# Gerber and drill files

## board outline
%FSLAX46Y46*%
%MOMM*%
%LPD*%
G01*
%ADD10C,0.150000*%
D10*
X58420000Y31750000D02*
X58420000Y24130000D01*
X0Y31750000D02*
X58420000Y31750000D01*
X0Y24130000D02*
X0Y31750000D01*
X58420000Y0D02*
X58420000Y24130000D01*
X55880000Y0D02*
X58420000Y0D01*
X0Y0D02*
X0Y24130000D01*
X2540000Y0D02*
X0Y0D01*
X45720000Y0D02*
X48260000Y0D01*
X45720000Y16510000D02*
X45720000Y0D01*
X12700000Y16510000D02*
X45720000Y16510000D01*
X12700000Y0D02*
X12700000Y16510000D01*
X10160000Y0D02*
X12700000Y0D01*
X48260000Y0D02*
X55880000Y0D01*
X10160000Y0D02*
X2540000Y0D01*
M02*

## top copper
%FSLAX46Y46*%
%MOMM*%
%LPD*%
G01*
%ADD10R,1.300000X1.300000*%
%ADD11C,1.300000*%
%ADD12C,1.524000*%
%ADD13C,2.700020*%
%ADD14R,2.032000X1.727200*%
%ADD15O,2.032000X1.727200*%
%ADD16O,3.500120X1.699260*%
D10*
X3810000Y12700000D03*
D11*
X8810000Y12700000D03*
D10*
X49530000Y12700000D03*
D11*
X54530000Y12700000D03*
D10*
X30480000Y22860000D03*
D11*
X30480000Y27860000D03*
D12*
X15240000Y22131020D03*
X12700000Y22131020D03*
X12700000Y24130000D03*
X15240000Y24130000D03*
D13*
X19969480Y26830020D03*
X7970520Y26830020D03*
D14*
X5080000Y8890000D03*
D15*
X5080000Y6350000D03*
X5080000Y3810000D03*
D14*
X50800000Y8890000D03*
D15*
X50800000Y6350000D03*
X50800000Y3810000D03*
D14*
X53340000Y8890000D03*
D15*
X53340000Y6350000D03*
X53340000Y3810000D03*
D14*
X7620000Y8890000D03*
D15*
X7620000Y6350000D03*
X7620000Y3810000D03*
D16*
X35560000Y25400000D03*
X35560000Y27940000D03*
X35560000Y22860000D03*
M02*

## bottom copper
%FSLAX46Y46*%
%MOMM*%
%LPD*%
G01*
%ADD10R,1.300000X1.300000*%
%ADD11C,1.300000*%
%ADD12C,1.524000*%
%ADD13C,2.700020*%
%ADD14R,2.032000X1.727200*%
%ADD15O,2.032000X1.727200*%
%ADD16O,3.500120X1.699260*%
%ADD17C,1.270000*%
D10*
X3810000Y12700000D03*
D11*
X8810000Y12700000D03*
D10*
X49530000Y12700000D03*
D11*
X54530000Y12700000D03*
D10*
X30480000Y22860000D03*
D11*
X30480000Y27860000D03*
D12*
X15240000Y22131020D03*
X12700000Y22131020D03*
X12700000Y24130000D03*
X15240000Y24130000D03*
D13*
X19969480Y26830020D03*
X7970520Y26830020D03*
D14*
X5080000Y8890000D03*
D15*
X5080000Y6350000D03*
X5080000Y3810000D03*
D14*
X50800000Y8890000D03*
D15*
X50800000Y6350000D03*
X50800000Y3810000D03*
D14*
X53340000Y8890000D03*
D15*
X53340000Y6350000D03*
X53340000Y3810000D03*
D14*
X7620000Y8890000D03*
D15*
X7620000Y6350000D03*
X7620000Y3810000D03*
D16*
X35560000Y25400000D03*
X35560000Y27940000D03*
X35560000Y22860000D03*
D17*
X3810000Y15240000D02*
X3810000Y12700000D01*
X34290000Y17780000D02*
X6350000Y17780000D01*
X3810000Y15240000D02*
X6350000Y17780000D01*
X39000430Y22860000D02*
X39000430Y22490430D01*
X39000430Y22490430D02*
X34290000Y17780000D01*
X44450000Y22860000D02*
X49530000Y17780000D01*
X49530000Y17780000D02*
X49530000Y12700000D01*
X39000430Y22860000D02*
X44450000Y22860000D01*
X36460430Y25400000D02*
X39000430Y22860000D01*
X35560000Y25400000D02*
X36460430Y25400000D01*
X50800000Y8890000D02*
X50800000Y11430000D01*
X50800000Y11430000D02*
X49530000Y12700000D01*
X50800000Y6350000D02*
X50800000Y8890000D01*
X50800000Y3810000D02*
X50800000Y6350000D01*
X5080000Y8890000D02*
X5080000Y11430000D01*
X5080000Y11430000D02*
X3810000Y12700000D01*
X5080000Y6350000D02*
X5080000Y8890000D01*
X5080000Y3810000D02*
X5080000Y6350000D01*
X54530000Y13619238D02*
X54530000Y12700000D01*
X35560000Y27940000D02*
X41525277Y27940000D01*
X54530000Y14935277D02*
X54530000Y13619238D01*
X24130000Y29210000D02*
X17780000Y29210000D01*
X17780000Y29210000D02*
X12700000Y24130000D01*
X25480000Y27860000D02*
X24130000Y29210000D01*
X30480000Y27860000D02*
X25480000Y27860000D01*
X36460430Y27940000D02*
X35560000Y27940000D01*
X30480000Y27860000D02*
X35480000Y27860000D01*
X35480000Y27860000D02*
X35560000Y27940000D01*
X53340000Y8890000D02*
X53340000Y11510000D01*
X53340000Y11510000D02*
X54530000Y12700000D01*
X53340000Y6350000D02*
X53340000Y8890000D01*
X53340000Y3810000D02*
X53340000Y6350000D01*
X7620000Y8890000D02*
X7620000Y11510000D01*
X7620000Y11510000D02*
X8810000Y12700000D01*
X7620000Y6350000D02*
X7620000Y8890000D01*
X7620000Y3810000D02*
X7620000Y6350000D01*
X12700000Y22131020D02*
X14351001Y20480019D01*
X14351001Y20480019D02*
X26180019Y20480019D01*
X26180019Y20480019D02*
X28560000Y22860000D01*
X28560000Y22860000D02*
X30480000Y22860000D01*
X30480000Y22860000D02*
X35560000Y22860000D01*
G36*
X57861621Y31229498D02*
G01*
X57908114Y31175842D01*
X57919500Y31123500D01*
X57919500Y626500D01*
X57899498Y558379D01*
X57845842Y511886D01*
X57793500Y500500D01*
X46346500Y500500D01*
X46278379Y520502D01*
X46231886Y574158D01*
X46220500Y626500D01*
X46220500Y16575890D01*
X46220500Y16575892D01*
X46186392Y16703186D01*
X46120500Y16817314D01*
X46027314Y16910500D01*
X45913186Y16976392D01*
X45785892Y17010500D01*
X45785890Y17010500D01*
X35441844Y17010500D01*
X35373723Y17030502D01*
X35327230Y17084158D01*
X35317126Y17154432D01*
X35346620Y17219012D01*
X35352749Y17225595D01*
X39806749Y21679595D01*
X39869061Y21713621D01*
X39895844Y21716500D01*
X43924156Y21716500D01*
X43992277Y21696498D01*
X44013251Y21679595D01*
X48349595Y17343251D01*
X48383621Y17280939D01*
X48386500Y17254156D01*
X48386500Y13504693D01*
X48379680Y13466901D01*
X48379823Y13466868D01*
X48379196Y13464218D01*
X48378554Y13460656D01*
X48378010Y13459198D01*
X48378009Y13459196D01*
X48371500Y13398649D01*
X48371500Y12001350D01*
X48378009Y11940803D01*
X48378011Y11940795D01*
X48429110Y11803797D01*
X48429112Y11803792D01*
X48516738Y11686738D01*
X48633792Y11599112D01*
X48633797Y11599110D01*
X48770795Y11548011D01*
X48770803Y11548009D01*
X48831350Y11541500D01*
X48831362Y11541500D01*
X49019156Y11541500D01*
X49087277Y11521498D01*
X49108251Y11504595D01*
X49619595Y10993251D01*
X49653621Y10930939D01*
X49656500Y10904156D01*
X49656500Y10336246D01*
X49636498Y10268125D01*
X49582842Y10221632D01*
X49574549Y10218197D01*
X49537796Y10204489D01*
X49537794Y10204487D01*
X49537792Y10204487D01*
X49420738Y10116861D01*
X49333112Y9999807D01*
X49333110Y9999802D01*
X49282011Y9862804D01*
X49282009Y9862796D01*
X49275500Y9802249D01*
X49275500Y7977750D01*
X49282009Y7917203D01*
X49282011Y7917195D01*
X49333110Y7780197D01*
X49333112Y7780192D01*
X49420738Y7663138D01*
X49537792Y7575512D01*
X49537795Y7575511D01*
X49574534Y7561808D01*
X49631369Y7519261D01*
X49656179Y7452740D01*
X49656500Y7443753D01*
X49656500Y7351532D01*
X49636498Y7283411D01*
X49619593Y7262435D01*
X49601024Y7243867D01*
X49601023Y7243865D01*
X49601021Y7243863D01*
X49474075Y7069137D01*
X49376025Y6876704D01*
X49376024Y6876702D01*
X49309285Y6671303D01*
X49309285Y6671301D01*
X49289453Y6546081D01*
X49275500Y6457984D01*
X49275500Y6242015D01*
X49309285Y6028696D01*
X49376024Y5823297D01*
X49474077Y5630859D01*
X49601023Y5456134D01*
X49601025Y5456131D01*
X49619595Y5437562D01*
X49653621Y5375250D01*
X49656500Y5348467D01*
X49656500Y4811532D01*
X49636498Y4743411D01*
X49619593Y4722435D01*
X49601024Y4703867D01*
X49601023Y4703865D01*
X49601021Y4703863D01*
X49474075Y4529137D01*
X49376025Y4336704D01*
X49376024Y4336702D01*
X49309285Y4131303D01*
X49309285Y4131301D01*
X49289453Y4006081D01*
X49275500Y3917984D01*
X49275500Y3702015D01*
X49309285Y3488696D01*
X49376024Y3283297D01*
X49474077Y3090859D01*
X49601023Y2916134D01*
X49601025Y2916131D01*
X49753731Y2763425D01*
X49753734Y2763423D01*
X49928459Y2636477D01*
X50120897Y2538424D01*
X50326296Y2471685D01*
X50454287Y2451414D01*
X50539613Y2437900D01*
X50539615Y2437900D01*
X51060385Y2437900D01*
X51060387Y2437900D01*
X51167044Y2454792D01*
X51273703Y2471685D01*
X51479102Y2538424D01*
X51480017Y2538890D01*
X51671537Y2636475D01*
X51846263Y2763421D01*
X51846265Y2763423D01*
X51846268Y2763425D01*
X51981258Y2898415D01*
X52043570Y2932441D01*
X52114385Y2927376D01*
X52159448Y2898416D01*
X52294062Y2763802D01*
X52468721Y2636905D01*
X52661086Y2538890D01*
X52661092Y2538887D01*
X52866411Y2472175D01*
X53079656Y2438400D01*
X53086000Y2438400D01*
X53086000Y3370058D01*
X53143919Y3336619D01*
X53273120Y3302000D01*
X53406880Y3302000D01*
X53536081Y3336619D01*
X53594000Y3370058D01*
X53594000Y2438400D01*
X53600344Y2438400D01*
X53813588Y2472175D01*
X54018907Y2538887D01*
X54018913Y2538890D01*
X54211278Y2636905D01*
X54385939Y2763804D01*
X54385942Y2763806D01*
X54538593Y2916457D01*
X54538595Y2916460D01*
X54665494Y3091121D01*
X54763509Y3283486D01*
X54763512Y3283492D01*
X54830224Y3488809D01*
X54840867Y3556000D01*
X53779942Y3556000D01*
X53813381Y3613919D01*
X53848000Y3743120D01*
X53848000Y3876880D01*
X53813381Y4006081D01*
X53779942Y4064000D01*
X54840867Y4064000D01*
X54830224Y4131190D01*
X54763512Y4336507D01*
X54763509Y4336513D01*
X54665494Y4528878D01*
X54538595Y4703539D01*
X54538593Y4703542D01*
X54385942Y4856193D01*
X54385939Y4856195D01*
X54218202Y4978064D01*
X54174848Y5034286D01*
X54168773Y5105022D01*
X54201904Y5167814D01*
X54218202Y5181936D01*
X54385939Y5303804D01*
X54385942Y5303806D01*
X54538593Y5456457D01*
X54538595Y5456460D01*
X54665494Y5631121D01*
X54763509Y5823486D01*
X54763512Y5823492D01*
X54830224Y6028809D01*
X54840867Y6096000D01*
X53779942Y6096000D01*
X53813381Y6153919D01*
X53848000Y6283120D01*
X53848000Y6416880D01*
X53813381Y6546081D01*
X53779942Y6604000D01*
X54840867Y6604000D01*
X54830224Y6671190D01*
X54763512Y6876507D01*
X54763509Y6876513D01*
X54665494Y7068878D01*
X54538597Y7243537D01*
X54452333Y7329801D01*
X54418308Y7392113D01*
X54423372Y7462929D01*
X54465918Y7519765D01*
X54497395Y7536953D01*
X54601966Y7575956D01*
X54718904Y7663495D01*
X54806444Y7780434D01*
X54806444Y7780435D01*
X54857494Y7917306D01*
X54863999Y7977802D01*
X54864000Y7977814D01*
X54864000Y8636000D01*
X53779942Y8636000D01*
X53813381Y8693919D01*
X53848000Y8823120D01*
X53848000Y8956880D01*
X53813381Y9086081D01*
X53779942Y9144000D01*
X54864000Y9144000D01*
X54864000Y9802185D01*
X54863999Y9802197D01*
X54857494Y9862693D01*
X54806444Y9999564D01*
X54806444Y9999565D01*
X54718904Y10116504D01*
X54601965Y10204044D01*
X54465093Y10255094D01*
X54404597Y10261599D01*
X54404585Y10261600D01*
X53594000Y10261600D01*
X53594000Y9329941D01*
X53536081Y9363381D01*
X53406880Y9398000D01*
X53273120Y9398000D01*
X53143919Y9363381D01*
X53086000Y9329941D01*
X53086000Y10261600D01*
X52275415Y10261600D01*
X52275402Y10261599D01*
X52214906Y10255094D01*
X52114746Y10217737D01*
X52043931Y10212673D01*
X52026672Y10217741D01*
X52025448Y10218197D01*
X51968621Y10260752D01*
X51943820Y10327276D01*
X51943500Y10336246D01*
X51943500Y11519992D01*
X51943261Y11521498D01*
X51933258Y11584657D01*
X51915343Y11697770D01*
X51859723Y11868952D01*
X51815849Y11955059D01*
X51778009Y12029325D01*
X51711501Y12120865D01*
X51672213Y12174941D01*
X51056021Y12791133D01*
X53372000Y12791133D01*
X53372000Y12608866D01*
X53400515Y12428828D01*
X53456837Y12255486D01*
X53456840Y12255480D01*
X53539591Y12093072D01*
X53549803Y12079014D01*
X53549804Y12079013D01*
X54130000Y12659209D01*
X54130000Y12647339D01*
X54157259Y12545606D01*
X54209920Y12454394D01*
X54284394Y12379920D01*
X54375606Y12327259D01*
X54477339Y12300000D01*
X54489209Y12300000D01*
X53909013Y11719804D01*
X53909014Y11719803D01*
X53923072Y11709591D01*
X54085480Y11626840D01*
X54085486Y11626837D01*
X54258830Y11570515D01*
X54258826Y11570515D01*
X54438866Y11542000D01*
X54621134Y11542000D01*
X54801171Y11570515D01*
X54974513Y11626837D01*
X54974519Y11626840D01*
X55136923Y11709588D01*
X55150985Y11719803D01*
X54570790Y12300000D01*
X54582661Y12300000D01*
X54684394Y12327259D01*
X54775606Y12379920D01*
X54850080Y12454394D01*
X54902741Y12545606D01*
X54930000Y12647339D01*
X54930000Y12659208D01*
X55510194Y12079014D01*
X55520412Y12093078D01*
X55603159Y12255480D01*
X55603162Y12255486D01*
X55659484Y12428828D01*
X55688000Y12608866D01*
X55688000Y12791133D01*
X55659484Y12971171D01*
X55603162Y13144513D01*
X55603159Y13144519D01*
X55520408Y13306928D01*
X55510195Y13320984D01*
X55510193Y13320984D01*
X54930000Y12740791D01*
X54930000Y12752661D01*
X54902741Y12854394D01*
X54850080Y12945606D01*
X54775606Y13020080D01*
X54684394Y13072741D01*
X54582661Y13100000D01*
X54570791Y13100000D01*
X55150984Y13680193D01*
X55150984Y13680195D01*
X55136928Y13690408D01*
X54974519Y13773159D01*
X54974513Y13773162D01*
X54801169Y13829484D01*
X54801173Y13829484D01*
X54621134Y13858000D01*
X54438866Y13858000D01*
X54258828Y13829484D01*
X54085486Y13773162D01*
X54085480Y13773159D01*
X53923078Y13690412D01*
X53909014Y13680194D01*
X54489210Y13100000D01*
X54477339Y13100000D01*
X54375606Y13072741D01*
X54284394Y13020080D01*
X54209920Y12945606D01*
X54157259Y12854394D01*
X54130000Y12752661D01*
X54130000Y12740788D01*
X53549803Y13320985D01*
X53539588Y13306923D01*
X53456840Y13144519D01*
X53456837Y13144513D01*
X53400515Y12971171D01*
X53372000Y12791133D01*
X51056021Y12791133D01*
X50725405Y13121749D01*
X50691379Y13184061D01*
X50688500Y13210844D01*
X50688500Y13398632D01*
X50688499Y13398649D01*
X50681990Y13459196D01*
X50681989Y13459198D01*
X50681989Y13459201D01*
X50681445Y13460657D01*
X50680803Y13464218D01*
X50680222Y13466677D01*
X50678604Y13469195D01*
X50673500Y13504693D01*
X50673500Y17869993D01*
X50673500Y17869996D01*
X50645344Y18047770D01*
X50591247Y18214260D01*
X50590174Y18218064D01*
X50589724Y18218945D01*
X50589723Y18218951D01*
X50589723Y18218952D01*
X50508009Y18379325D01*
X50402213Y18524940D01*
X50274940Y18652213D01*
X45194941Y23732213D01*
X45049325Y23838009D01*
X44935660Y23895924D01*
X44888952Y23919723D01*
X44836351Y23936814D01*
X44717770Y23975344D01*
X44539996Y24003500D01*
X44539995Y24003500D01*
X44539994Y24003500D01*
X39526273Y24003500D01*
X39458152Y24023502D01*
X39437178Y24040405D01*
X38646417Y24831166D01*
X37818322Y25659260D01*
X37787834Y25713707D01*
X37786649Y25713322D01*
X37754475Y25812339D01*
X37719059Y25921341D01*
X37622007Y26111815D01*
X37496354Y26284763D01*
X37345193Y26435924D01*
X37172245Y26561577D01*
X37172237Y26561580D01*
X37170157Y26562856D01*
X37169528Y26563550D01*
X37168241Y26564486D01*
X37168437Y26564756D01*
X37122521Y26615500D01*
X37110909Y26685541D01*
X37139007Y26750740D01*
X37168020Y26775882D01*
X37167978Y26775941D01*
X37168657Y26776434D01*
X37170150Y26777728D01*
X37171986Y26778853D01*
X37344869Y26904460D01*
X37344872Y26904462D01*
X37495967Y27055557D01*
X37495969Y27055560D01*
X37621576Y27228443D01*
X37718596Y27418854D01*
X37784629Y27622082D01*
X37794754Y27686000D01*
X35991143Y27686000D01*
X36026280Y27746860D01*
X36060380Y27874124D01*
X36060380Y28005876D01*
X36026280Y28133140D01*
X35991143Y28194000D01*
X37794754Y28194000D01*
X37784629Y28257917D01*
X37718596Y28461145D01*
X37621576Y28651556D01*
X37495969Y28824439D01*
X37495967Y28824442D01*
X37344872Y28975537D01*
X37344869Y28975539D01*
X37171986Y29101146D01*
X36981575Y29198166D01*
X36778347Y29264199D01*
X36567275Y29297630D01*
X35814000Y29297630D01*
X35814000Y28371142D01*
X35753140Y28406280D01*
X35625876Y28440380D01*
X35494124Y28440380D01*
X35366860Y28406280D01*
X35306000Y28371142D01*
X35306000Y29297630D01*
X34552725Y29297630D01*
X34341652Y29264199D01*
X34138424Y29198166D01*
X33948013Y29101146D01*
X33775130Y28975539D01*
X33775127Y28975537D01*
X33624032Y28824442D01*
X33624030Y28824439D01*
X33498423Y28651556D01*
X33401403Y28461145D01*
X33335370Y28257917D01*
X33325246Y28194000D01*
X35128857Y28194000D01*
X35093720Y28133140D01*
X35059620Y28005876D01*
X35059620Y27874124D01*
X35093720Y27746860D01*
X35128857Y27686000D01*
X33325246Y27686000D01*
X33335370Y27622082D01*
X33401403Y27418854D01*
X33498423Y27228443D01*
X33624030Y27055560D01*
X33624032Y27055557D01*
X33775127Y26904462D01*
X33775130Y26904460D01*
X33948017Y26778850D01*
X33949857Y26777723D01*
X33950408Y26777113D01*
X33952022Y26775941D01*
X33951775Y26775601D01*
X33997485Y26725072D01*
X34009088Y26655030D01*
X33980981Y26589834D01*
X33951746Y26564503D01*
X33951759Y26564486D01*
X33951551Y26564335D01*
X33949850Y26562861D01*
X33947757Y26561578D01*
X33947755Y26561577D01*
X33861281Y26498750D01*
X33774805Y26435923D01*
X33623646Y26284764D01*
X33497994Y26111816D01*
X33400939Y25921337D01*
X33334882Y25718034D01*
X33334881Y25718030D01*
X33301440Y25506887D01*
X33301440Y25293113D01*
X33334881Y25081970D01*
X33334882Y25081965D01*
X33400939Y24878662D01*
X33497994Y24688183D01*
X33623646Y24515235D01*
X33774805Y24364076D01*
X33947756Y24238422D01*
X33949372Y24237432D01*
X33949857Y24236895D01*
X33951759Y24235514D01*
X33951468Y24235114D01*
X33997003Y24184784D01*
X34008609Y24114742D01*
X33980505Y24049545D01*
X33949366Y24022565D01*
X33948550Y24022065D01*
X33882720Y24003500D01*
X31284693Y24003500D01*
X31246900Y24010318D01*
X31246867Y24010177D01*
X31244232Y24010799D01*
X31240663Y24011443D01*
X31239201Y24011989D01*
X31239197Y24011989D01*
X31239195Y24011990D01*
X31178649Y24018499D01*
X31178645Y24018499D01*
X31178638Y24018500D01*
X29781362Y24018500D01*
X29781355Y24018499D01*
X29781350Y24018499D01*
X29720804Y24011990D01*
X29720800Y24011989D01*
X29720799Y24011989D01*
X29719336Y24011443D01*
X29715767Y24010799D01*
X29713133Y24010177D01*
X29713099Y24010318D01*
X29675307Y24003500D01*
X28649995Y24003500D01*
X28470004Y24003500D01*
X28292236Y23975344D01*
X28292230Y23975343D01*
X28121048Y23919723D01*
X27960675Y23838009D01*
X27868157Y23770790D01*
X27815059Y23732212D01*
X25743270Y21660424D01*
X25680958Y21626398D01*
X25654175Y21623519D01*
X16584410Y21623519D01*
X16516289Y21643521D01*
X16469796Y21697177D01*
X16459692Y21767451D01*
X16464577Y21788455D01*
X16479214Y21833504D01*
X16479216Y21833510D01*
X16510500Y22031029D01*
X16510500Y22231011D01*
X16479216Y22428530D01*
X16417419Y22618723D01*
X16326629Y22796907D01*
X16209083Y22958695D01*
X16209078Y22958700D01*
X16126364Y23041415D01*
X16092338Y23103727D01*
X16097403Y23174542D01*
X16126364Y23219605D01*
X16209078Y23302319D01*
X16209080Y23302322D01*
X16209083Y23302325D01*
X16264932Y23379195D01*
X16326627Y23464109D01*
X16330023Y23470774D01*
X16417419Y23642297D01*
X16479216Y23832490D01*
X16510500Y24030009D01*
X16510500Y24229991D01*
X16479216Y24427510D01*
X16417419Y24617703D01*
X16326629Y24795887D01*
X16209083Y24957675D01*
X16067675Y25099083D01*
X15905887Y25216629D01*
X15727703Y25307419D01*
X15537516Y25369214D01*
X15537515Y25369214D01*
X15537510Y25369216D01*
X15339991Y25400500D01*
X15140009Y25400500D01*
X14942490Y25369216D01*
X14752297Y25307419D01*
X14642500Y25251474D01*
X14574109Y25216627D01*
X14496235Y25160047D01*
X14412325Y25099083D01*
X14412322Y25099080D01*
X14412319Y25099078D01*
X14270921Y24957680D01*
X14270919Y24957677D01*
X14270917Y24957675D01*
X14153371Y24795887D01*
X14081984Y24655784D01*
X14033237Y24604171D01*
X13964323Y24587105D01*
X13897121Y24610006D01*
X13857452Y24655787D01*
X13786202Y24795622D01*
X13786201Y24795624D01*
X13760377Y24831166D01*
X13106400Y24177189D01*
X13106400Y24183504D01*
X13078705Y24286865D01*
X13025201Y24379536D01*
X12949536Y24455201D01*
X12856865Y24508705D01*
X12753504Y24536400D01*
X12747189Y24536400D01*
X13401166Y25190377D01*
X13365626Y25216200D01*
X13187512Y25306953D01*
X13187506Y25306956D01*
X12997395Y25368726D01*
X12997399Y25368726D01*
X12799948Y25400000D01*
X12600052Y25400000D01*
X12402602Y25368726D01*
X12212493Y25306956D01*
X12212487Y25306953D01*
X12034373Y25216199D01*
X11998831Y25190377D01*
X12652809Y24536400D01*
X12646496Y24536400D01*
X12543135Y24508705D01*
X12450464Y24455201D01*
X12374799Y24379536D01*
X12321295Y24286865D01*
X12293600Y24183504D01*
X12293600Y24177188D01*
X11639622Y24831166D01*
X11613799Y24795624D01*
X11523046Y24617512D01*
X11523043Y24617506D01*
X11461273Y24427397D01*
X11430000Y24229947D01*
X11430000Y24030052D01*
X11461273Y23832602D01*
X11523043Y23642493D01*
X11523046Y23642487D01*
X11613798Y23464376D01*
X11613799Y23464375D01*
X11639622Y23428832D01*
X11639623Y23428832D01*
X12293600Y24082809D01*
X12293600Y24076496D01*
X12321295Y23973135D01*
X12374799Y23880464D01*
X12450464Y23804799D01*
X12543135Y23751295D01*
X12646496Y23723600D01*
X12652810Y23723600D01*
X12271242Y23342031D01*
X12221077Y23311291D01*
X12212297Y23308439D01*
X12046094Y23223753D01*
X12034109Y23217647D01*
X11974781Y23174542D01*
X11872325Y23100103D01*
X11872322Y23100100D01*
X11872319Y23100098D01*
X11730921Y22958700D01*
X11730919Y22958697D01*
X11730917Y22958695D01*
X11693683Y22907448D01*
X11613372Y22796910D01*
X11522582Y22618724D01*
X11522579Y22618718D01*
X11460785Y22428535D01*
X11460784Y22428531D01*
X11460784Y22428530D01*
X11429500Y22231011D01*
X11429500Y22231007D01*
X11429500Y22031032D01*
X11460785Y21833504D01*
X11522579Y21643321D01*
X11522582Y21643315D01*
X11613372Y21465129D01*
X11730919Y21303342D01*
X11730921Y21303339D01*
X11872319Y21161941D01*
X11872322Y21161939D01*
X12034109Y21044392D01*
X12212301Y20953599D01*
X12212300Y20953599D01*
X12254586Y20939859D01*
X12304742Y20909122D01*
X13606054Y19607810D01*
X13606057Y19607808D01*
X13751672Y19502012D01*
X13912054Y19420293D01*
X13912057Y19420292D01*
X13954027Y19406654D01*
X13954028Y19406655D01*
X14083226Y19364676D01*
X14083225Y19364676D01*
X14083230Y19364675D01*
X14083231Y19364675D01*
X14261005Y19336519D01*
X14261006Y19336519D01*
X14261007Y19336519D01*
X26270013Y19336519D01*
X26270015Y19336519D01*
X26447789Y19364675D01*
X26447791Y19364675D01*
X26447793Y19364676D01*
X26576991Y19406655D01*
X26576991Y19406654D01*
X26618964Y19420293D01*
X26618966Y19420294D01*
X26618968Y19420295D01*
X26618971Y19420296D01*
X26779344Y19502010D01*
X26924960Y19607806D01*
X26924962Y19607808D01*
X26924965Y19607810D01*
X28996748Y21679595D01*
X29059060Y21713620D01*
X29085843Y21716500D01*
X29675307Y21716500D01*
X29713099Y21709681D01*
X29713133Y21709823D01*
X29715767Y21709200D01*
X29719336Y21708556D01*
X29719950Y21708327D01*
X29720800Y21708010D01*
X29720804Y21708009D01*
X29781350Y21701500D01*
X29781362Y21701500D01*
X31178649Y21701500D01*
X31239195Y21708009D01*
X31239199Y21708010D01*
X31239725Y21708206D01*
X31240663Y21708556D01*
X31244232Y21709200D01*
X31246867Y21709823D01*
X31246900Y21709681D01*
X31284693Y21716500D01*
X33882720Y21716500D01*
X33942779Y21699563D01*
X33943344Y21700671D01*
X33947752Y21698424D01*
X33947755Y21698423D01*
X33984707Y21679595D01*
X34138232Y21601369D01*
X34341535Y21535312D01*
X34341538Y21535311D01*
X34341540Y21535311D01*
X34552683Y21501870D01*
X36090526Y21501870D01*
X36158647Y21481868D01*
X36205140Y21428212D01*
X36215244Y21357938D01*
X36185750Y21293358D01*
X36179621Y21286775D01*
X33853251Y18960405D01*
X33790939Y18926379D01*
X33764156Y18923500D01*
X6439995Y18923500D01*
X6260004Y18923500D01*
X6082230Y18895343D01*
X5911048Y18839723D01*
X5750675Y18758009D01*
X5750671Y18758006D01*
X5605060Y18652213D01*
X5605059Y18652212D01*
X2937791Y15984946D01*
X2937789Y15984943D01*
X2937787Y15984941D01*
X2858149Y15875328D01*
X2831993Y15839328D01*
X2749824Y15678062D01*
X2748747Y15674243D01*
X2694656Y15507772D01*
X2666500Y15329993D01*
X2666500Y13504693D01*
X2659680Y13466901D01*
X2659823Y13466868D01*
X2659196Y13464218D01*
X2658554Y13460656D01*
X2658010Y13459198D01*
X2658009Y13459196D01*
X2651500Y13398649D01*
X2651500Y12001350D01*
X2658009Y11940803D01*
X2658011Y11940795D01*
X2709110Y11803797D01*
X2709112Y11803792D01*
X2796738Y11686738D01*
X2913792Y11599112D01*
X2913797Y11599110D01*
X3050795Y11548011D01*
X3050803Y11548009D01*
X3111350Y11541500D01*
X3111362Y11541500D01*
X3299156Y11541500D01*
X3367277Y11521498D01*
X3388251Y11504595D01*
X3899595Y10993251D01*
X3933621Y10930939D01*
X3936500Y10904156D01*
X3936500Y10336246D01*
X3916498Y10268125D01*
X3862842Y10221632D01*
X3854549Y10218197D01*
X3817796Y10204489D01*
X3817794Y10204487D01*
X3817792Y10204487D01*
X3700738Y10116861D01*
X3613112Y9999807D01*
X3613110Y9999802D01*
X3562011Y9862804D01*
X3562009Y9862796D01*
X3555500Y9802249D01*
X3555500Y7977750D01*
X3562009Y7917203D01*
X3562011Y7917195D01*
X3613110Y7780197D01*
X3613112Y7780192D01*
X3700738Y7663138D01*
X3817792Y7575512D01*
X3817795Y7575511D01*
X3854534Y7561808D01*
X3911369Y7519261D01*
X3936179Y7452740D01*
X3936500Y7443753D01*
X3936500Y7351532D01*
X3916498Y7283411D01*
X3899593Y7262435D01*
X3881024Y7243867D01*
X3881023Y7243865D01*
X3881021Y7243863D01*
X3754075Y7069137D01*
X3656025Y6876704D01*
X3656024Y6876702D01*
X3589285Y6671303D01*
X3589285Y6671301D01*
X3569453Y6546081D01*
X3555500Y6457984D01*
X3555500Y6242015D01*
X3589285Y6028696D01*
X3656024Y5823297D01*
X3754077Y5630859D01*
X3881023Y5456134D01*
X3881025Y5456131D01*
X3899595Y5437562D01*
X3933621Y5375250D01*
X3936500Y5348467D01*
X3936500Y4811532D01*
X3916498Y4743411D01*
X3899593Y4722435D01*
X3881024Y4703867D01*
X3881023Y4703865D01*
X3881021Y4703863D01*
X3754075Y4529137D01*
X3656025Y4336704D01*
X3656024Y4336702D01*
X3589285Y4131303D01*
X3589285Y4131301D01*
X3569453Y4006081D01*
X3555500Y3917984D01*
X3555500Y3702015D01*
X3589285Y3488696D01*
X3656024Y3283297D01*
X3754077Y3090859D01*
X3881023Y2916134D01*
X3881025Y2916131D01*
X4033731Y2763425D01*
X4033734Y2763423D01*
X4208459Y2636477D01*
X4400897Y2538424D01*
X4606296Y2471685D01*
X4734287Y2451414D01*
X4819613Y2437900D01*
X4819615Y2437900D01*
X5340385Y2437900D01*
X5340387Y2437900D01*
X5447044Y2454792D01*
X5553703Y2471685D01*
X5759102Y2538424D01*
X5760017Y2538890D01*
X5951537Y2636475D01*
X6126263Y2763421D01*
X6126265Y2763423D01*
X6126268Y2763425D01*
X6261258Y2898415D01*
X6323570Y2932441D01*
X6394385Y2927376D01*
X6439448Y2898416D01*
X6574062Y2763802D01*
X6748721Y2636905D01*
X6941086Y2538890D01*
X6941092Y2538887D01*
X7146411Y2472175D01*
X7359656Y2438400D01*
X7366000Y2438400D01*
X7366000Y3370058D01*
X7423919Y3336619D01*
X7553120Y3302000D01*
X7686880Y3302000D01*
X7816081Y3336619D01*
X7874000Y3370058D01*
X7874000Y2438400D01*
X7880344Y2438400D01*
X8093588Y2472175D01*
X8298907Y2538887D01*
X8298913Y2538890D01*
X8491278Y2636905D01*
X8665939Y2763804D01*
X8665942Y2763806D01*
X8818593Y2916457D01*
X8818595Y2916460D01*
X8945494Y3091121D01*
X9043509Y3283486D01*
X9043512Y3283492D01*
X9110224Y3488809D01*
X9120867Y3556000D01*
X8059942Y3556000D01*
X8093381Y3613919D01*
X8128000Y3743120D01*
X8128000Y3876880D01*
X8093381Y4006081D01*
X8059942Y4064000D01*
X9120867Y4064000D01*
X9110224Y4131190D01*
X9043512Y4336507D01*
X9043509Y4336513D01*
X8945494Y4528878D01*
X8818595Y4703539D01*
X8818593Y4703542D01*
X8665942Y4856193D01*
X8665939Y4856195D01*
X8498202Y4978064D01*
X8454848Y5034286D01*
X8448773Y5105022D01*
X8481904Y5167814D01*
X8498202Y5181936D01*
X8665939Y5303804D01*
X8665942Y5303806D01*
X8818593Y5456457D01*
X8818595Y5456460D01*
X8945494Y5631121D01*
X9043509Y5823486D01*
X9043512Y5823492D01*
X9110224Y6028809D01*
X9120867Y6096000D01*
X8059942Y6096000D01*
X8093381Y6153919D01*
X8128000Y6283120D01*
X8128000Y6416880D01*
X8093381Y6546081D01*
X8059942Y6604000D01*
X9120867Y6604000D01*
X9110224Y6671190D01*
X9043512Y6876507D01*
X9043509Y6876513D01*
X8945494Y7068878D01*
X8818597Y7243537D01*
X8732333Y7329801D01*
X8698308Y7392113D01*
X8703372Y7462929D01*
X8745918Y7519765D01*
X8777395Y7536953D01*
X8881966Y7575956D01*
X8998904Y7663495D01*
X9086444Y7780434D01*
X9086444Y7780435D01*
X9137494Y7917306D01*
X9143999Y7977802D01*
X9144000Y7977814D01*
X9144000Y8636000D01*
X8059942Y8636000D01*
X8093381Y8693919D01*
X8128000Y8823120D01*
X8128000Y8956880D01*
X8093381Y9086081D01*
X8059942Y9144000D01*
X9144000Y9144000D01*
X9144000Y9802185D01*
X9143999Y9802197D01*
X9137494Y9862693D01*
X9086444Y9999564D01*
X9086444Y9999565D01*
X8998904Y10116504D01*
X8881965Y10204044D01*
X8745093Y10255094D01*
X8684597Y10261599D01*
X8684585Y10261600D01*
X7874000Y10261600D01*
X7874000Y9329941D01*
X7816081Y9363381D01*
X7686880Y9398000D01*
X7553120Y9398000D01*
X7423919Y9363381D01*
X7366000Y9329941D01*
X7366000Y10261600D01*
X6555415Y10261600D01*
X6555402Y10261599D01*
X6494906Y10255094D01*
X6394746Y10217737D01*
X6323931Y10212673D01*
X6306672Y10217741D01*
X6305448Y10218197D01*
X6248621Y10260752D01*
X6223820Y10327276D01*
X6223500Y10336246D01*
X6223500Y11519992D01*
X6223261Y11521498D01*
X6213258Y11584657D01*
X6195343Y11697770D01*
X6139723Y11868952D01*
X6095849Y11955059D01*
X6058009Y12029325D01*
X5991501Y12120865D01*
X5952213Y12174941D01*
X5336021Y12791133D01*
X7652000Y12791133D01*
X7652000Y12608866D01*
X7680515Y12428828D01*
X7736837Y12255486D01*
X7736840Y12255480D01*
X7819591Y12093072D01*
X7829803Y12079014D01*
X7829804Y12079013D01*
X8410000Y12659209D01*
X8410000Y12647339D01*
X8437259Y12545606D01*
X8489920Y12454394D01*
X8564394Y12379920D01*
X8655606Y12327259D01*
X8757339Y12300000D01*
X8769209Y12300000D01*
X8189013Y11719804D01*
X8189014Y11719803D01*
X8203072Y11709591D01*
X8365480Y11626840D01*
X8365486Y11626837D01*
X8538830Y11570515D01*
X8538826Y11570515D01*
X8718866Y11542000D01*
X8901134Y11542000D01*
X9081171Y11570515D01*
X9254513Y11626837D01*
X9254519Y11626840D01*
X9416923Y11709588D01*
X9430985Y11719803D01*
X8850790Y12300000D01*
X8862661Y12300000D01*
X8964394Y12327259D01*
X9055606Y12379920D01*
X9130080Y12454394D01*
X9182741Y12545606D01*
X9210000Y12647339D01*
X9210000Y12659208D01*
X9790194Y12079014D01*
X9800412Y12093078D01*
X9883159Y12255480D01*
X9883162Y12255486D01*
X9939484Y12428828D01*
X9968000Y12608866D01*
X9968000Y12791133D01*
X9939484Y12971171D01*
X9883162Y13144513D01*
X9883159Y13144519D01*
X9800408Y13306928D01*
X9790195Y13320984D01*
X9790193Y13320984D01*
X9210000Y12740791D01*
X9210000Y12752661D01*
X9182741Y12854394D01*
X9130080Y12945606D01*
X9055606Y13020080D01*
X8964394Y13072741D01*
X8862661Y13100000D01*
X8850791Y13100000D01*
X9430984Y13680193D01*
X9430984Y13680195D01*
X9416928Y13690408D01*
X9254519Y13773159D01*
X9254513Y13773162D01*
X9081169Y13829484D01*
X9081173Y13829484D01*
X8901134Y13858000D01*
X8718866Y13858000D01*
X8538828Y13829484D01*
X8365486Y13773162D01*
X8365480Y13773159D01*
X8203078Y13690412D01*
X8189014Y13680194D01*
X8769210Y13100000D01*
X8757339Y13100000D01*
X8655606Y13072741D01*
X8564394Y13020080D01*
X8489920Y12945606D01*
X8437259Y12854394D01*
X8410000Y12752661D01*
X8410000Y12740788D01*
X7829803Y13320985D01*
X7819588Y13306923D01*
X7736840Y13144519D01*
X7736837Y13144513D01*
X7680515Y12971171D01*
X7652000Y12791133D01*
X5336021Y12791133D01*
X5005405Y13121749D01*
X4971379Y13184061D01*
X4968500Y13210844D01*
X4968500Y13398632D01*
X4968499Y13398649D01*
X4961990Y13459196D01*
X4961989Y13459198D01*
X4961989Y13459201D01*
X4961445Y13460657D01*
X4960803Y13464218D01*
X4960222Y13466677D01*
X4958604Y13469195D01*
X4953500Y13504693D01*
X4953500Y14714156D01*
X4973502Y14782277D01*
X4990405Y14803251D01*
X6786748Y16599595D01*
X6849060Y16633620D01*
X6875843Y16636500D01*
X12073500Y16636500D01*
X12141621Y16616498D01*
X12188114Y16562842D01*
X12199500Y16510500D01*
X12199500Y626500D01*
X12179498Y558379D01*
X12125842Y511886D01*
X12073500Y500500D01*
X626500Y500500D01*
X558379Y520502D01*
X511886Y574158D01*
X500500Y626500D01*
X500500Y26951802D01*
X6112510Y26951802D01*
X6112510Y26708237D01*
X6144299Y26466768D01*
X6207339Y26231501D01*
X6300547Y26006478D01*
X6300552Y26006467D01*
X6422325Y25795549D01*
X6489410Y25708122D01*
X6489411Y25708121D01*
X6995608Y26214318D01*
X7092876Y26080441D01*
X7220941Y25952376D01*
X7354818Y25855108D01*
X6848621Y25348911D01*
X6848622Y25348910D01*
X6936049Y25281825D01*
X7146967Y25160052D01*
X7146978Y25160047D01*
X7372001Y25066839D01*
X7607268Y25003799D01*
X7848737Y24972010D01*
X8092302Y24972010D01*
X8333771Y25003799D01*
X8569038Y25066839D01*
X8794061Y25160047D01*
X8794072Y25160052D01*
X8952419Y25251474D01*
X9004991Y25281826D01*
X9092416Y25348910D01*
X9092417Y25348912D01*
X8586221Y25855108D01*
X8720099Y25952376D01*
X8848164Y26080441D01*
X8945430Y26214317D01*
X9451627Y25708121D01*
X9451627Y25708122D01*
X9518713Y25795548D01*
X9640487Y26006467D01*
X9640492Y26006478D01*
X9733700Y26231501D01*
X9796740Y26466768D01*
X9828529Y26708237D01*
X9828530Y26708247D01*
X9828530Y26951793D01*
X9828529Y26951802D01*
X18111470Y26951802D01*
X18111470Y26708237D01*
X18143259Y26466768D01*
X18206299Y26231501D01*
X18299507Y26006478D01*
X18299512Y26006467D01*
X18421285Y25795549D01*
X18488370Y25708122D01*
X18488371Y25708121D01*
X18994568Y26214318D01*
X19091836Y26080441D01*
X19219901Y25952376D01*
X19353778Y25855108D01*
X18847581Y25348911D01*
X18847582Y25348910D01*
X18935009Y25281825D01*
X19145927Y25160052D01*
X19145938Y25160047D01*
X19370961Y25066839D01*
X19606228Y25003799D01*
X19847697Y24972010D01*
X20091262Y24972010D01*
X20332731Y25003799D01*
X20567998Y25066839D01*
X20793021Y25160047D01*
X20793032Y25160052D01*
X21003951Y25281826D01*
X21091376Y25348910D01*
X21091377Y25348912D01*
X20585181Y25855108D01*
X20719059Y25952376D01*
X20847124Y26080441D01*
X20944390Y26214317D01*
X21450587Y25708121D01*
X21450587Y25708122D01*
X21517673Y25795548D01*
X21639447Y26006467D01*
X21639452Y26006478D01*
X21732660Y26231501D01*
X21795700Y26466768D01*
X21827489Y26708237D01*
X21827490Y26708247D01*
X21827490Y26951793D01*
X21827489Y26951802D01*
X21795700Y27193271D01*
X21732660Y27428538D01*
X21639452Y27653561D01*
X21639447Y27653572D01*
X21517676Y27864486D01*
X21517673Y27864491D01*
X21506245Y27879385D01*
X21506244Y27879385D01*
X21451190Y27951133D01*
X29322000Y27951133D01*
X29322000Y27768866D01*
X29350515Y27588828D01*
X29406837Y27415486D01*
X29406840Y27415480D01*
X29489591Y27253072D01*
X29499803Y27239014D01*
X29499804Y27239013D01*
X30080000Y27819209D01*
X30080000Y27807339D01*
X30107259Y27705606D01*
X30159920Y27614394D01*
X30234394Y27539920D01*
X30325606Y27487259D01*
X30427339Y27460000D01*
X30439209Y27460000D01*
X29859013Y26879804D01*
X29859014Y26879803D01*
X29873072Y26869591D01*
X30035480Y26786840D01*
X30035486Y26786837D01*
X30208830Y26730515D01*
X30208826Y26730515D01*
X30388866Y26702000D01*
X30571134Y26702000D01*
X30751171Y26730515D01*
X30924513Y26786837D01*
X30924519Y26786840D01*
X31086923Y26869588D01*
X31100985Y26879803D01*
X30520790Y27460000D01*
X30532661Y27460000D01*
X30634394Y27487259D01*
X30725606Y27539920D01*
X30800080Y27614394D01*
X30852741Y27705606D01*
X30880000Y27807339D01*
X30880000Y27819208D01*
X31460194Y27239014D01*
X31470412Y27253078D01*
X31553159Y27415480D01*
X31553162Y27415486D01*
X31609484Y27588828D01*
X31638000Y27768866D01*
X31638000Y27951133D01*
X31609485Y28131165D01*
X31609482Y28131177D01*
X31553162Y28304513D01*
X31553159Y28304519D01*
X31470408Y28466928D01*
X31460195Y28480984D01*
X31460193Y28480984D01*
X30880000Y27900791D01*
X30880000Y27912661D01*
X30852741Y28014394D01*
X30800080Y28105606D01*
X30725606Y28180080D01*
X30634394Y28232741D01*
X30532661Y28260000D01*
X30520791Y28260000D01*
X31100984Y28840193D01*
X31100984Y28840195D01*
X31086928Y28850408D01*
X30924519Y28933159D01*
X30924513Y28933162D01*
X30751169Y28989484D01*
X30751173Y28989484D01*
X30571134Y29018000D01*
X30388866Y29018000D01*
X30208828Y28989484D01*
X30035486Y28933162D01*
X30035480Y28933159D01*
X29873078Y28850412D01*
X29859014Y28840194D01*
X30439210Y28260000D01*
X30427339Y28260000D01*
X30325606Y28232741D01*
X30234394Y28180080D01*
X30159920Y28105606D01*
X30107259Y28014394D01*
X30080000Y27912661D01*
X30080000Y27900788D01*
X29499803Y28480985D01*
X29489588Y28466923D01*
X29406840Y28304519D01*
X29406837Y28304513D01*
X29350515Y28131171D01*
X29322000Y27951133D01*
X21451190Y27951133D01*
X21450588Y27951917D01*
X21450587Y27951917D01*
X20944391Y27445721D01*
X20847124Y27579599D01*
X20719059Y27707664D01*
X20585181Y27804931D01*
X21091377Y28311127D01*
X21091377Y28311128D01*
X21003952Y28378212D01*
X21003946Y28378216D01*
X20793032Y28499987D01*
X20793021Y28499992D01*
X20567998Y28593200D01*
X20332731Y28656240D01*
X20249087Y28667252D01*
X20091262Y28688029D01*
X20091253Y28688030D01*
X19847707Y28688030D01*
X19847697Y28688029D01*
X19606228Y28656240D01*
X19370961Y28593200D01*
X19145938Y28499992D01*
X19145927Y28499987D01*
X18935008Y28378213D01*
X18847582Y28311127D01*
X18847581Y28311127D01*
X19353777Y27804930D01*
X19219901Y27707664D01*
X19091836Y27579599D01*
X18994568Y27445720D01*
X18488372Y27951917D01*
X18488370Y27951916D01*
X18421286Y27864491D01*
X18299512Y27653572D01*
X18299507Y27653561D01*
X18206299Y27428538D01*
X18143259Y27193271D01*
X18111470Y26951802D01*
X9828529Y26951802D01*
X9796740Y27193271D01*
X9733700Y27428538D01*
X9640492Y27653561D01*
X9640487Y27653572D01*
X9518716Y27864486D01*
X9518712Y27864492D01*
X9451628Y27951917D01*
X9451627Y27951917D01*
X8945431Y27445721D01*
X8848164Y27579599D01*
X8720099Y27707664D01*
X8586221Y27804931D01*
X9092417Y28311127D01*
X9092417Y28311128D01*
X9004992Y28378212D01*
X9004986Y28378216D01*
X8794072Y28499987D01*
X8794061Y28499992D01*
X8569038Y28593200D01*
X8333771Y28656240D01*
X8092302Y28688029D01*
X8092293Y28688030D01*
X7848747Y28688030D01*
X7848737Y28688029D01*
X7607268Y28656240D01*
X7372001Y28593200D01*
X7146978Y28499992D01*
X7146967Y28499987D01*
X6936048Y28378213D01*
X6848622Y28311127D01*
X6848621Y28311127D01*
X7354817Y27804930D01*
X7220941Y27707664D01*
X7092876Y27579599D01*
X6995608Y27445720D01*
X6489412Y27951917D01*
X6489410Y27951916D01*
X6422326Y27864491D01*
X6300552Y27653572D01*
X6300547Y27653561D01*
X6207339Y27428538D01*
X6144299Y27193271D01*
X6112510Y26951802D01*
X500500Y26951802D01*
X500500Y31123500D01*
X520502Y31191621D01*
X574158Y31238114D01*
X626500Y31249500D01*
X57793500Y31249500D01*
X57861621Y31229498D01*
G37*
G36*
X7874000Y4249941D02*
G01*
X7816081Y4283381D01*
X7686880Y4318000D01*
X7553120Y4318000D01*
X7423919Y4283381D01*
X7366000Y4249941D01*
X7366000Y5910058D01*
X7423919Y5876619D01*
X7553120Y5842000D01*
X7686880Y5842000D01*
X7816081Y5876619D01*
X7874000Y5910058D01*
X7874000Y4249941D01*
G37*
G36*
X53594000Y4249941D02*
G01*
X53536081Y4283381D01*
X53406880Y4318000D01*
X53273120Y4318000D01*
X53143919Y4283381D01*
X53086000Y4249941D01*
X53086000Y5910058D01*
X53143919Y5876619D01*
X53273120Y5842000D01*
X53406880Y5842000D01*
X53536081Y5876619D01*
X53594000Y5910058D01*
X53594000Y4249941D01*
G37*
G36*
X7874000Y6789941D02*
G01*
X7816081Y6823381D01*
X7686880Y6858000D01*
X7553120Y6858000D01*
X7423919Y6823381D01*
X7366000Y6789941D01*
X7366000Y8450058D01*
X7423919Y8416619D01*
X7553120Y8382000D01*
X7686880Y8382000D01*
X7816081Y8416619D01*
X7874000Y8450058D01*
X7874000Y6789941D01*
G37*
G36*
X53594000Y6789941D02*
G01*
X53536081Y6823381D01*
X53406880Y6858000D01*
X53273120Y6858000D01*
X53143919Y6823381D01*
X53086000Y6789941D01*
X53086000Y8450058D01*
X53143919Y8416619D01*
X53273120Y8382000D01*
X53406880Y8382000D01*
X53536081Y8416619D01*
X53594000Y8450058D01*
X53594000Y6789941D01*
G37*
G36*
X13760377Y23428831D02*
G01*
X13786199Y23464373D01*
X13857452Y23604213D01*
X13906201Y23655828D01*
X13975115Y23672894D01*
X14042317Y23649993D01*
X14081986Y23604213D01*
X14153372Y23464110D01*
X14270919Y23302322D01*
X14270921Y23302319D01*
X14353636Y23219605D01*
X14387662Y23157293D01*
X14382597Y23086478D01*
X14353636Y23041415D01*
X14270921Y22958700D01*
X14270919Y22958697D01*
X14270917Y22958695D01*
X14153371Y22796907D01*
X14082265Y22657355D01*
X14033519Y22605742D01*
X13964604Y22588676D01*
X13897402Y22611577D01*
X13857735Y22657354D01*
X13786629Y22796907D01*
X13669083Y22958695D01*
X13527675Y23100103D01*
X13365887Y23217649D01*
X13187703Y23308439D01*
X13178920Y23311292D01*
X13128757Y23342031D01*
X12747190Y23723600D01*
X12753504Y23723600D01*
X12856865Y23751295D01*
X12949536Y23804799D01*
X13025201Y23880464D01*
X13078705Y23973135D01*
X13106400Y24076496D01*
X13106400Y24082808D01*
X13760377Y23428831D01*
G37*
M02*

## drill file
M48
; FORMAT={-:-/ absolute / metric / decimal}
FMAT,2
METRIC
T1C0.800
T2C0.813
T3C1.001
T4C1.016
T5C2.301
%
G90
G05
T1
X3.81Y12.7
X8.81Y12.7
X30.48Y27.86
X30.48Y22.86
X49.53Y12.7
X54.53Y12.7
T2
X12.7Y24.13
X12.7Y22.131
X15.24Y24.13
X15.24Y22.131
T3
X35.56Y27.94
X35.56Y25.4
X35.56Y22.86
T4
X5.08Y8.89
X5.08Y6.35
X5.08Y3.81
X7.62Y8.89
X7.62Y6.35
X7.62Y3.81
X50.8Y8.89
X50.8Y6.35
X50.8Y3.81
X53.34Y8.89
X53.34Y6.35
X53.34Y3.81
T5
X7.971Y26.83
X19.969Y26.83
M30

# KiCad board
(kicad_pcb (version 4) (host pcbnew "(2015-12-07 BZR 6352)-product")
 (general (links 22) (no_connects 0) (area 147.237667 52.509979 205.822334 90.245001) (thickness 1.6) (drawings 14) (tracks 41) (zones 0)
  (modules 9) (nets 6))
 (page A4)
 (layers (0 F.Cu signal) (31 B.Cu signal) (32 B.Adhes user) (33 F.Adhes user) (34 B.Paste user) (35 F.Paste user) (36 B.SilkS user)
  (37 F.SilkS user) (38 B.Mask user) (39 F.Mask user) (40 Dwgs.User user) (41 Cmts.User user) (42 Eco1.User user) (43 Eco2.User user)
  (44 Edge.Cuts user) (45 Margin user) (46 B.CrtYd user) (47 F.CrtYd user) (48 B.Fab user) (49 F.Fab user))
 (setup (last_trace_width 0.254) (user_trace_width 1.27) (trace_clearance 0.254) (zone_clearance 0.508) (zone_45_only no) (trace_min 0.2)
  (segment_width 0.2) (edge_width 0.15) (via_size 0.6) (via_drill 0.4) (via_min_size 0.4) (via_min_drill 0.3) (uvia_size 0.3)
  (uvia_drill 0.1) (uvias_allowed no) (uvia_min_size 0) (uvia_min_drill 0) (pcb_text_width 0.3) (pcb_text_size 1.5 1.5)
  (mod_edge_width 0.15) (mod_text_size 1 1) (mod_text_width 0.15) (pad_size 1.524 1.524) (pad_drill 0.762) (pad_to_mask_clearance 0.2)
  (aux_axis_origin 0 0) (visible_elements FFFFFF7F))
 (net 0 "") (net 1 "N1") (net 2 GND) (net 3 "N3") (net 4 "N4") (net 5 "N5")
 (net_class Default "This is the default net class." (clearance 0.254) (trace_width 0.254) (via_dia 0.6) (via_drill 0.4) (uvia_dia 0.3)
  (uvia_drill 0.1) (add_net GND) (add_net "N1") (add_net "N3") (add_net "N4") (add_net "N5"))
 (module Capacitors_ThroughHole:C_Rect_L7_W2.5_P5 (layer F.Cu) (at 3.81 -12.7)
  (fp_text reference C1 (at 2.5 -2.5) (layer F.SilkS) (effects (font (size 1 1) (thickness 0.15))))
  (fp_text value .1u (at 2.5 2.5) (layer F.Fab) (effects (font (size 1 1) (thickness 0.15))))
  (pad 1 thru_hole rect (at 0 0) (size 1.3 1.3) (drill 0.8) (layers *.Cu *.Mask F.SilkS) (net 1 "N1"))
  (pad 2 thru_hole circle (at 5 0) (size 1.3 1.3) (drill 0.8) (layers *.Cu *.Mask F.SilkS) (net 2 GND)))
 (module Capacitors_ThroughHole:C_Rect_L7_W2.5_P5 (layer F.Cu) (at 49.53 -12.7)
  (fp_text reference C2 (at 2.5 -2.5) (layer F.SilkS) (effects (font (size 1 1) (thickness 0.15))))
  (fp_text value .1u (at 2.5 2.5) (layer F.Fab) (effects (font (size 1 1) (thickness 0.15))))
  (pad 1 thru_hole rect (at 0 0) (size 1.3 1.3) (drill 0.8) (layers *.Cu *.Mask F.SilkS) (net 1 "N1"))
  (pad 2 thru_hole circle (at 5 0) (size 1.3 1.3) (drill 0.8) (layers *.Cu *.Mask F.SilkS) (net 2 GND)))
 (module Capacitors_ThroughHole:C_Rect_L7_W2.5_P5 (layer F.Cu) (at 30.48 -22.86 90)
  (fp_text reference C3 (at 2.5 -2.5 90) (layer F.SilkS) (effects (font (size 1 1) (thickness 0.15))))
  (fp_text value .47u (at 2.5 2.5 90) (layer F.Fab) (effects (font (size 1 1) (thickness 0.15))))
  (pad 1 thru_hole rect (at 0 0 90) (size 1.3 1.3) (drill 0.8) (layers *.Cu *.Mask F.SilkS) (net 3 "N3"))
  (pad 2 thru_hole circle (at 5 0 90) (size 1.3 1.3) (drill 0.8) (layers *.Cu *.Mask F.SilkS) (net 2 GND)))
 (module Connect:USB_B (layer F.Cu) (at 12.7 -22.13102 90)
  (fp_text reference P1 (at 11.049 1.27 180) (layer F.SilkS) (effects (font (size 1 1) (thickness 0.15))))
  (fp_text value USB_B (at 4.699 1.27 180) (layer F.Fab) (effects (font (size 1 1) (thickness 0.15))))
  (pad 2 thru_hole circle (at 0 2.54) (size 1.524 1.524) (drill 0.8128) (layers *.Cu *.Mask F.SilkS) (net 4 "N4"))
  (pad 1 thru_hole circle (at 0 0) (size 1.524 1.524) (drill 0.8128) (layers *.Cu *.Mask F.SilkS) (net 3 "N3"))
  (pad 4 thru_hole circle (at 1.99898 0) (size 1.524 1.524) (drill 0.8128) (layers *.Cu *.Mask F.SilkS) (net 2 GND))
  (pad 3 thru_hole circle (at 1.99898 2.54) (size 1.524 1.524) (drill 0.8128) (layers *.Cu *.Mask F.SilkS) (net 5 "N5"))
  (pad 5 thru_hole circle (at 4.699 7.26948) (size 2.70002 2.70002) (drill 2.30124) (layers *.Cu *.Mask F.SilkS) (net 2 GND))
  (pad 5 thru_hole circle (at 4.699 -4.72948) (size 2.70002 2.70002) (drill 2.30124) (layers *.Cu *.Mask F.SilkS) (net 2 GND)))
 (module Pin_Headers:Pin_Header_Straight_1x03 (layer F.Cu) (at 5.08 -8.89)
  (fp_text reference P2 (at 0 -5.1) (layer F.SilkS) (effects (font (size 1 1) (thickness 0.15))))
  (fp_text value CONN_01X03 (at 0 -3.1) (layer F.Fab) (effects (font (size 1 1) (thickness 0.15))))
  (pad 1 thru_hole rect (at 0 0) (size 2.032 1.7272) (drill 1.016) (layers *.Cu *.Mask F.SilkS) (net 1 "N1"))
  (pad 2 thru_hole oval (at 0 2.54) (size 2.032 1.7272) (drill 1.016) (layers *.Cu *.Mask F.SilkS) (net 1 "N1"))
  (pad 3 thru_hole oval (at 0 5.08) (size 2.032 1.7272) (drill 1.016) (layers *.Cu *.Mask F.SilkS) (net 1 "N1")))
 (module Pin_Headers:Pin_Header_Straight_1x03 (layer F.Cu) (at 50.8 -8.89)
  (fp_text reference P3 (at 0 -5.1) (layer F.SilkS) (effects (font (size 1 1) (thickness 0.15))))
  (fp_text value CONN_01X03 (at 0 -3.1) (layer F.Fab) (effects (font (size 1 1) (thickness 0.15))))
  (pad 1 thru_hole rect (at 0 0) (size 2.032 1.7272) (drill 1.016) (layers *.Cu *.Mask F.SilkS) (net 1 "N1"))
  (pad 2 thru_hole oval (at 0 2.54) (size 2.032 1.7272) (drill 1.016) (layers *.Cu *.Mask F.SilkS) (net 1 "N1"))
  (pad 3 thru_hole oval (at 0 5.08) (size 2.032 1.7272) (drill 1.016) (layers *.Cu *.Mask F.SilkS) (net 1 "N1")))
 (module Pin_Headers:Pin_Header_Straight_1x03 (layer F.Cu) (at 53.34 -8.89)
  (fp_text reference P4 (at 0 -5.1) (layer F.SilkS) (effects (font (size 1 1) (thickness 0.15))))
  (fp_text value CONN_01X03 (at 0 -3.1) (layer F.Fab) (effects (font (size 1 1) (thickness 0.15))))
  (pad 1 thru_hole rect (at 0 0) (size 2.032 1.7272) (drill 1.016) (layers *.Cu *.Mask F.SilkS) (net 2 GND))
  (pad 2 thru_hole oval (at 0 2.54) (size 2.032 1.7272) (drill 1.016) (layers *.Cu *.Mask F.SilkS) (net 2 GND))
  (pad 3 thru_hole oval (at 0 5.08) (size 2.032 1.7272) (drill 1.016) (layers *.Cu *.Mask F.SilkS) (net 2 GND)))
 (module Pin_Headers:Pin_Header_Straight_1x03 (layer F.Cu) (at 7.62 -8.89)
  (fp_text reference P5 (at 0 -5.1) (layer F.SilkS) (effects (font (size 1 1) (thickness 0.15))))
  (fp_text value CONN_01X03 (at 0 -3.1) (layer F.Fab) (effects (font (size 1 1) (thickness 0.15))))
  (pad 1 thru_hole rect (at 0 0) (size 2.032 1.7272) (drill 1.016) (layers *.Cu *.Mask F.SilkS) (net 2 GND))
  (pad 2 thru_hole oval (at 0 2.54) (size 2.032 1.7272) (drill 1.016) (layers *.Cu *.Mask F.SilkS) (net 2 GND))
  (pad 3 thru_hole oval (at 0 5.08) (size 2.032 1.7272) (drill 1.016) (layers *.Cu *.Mask F.SilkS) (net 2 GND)))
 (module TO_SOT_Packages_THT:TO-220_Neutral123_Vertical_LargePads (layer F.Cu) (at 35.56 -25.4 270)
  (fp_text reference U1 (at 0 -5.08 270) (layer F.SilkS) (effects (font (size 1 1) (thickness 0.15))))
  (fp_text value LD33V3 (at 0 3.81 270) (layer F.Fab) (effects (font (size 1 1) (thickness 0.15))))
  (pad 2 thru_hole oval (at 0 0) (size 3.50012 1.69926) (drill 1.00076) (layers *.Cu *.Mask F.SilkS) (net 1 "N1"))
  (pad 1 thru_hole oval (at -2.54 0) (size 3.50012 1.69926) (drill 1.00076) (layers *.Cu *.Mask F.SilkS) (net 2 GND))
  (pad 3 thru_hole oval (at 2.54 0) (size 3.50012 1.69926) (drill 1.00076) (layers *.Cu *.Mask F.SilkS) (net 3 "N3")))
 (gr_line (start 58.42 -31.75) (end 58.42 -24.13) (layer Edge.Cuts) (width 0.15))
 (gr_line (start 0 -31.75) (end 58.42 -31.75) (layer Edge.Cuts) (width 0.15))
 (gr_line (start 0 -24.13) (end 0 -31.75) (layer Edge.Cuts) (width 0.15))
 (gr_line (start 58.42 0) (end 58.42 -24.13) (layer Edge.Cuts) (width 0.15))
 (gr_line (start 55.88 0) (end 58.42 0) (layer Edge.Cuts) (width 0.15))
 (gr_line (start 0 0) (end 0 -24.13) (layer Edge.Cuts) (width 0.15))
 (gr_line (start 2.54 0) (end 0 0) (layer Edge.Cuts) (width 0.15))
 (gr_line (start 45.72 0) (end 48.26 0) (layer Edge.Cuts) (width 0.15))
 (gr_line (start 45.72 -16.51) (end 45.72 0) (layer Edge.Cuts) (width 0.15))
 (gr_line (start 12.7 -16.51) (end 45.72 -16.51) (layer Edge.Cuts) (width 0.15))
 (gr_line (start 12.7 0) (end 12.7 -16.51) (layer Edge.Cuts) (width 0.15))
 (gr_line (start 10.16 0) (end 12.7 0) (layer Edge.Cuts) (width 0.15))
 (gr_line (start 48.26 0) (end 55.88 0) (layer Edge.Cuts) (width 0.15))
 (gr_line (start 10.16 0) (end 2.54 0) (layer Edge.Cuts) (width 0.15))
 (segment (start 3.81 -15.24) (end 3.81 -12.7) (width 1.27) (layer B.Cu) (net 1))
 (segment (start 34.29 -17.78) (end 6.35 -17.78) (width 1.27) (layer B.Cu) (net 1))
 (segment (start 3.81 -15.24) (end 6.35 -17.78) (width 1.27) (layer B.Cu) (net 1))
 (segment (start 39.00043 -22.86) (end 39.00043 -22.49043) (width 1.27) (layer B.Cu) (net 1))
 (segment (start 39.00043 -22.49043) (end 34.29 -17.78) (width 1.27) (layer B.Cu) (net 1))
 (segment (start 44.45 -22.86) (end 49.53 -17.78) (width 1.27) (layer B.Cu) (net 1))
 (segment (start 49.53 -17.78) (end 49.53 -12.7) (width 1.27) (layer B.Cu) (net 1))
 (segment (start 39.00043 -22.86) (end 44.45 -22.86) (width 1.27) (layer B.Cu) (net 1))
 (segment (start 36.46043 -25.4) (end 39.00043 -22.86) (width 1.27) (layer B.Cu) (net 1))
 (segment (start 35.56 -25.4) (end 36.46043 -25.4) (width 1.27) (layer B.Cu) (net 1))
 (segment (start 50.8 -8.89) (end 50.8 -11.43) (width 1.27) (layer B.Cu) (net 1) (status 10))
 (segment (start 50.8 -11.43) (end 49.53 -12.7) (width 1.27) (layer B.Cu) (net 1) (status 20))
 (segment (start 50.8 -6.35) (end 50.8 -8.89) (width 1.27) (layer B.Cu) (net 1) (status 30))
 (segment (start 50.8 -3.81) (end 50.8 -6.35) (width 1.27) (layer B.Cu) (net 1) (status 30))
 (segment (start 5.08 -8.89) (end 5.08 -11.43) (width 1.27) (layer B.Cu) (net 1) (status 10))
 (segment (start 5.08 -11.43) (end 3.81 -12.7) (width 1.27) (layer B.Cu) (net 1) (status 20))
 (segment (start 5.08 -6.35) (end 5.08 -8.89) (width 1.27) (layer B.Cu) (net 1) (status 30))
 (segment (start 5.08 -3.81) (end 5.08 -6.35) (width 1.27) (layer B.Cu) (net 1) (status 30))
 (segment (start 54.53 -13.619238) (end 54.53 -12.7) (width 1.27) (layer B.Cu) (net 2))
 (segment (start 35.56 -27.94) (end 41.525277 -27.94) (width 1.27) (layer B.Cu) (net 2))
 (segment (start 54.53 -14.935277) (end 54.53 -13.619238) (width 1.27) (layer B.Cu) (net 2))
 (segment (start 24.13 -29.21) (end 17.78 -29.21) (width 1.27) (layer B.Cu) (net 2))
 (segment (start 17.78 -29.21) (end 12.7 -24.13) (width 1.27) (layer B.Cu) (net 2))
 (segment (start 25.48 -27.86) (end 24.13 -29.21) (width 1.27) (layer B.Cu) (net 2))
 (segment (start 30.48 -27.86) (end 25.48 -27.86) (width 1.27) (layer B.Cu) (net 2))
 (segment (start 36.46043 -27.94) (end 35.56 -27.94) (width 1.27) (layer B.Cu) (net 2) (status 30))
 (segment (start 30.48 -27.86) (end 35.48 -27.86) (width 1.27) (layer B.Cu) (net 2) (status 30))
 (segment (start 35.48 -27.86) (end 35.56 -27.94) (width 1.27) (layer B.Cu) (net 2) (status 30))
 (segment (start 53.34 -8.89) (end 53.34 -11.51) (width 1.27) (layer B.Cu) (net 2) (status 10))
 (segment (start 53.34 -11.51) (end 54.53 -12.7) (width 1.27) (layer B.Cu) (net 2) (status 20))
 (segment (start 53.34 -6.35) (end 53.34 -8.89) (width 1.27) (layer B.Cu) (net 2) (status 30))
 (segment (start 53.34 -3.81) (end 53.34 -6.35) (width 1.27) (layer B.Cu) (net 2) (status 30))
 (segment (start 7.62 -8.89) (end 7.62 -11.51) (width 1.27) (layer B.Cu) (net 2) (status 10))
 (segment (start 7.62 -11.51) (end 8.81 -12.7) (width 1.27) (layer B.Cu) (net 2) (status 20))
 (segment (start 7.62 -6.35) (end 7.62 -8.89) (width 1.27) (layer B.Cu) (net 2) (status 30))
 (segment (start 7.62 -3.81) (end 7.62 -6.35) (width 1.27) (layer B.Cu) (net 2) (status 30))
 (segment (start 12.7 -22.13102) (end 14.351001 -20.480019) (width 1.27) (layer B.Cu) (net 3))
 (segment (start 14.351001 -20.480019) (end 26.180019 -20.480019) (width 1.27) (layer B.Cu) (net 3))
 (segment (start 26.180019 -20.480019) (end 28.56 -22.86) (width 1.27) (layer B.Cu) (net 3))
 (segment (start 28.56 -22.86) (end 30.48 -22.86) (width 1.27) (layer B.Cu) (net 3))
 (segment (start 30.48 -22.86) (end 35.56 -22.86) (width 1.27) (layer B.Cu) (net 3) (status 30))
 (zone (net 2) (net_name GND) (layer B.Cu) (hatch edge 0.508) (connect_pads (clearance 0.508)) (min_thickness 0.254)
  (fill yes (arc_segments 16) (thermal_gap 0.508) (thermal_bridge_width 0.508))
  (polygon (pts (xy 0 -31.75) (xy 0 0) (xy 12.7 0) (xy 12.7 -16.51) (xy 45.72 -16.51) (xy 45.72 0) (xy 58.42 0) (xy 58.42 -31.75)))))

